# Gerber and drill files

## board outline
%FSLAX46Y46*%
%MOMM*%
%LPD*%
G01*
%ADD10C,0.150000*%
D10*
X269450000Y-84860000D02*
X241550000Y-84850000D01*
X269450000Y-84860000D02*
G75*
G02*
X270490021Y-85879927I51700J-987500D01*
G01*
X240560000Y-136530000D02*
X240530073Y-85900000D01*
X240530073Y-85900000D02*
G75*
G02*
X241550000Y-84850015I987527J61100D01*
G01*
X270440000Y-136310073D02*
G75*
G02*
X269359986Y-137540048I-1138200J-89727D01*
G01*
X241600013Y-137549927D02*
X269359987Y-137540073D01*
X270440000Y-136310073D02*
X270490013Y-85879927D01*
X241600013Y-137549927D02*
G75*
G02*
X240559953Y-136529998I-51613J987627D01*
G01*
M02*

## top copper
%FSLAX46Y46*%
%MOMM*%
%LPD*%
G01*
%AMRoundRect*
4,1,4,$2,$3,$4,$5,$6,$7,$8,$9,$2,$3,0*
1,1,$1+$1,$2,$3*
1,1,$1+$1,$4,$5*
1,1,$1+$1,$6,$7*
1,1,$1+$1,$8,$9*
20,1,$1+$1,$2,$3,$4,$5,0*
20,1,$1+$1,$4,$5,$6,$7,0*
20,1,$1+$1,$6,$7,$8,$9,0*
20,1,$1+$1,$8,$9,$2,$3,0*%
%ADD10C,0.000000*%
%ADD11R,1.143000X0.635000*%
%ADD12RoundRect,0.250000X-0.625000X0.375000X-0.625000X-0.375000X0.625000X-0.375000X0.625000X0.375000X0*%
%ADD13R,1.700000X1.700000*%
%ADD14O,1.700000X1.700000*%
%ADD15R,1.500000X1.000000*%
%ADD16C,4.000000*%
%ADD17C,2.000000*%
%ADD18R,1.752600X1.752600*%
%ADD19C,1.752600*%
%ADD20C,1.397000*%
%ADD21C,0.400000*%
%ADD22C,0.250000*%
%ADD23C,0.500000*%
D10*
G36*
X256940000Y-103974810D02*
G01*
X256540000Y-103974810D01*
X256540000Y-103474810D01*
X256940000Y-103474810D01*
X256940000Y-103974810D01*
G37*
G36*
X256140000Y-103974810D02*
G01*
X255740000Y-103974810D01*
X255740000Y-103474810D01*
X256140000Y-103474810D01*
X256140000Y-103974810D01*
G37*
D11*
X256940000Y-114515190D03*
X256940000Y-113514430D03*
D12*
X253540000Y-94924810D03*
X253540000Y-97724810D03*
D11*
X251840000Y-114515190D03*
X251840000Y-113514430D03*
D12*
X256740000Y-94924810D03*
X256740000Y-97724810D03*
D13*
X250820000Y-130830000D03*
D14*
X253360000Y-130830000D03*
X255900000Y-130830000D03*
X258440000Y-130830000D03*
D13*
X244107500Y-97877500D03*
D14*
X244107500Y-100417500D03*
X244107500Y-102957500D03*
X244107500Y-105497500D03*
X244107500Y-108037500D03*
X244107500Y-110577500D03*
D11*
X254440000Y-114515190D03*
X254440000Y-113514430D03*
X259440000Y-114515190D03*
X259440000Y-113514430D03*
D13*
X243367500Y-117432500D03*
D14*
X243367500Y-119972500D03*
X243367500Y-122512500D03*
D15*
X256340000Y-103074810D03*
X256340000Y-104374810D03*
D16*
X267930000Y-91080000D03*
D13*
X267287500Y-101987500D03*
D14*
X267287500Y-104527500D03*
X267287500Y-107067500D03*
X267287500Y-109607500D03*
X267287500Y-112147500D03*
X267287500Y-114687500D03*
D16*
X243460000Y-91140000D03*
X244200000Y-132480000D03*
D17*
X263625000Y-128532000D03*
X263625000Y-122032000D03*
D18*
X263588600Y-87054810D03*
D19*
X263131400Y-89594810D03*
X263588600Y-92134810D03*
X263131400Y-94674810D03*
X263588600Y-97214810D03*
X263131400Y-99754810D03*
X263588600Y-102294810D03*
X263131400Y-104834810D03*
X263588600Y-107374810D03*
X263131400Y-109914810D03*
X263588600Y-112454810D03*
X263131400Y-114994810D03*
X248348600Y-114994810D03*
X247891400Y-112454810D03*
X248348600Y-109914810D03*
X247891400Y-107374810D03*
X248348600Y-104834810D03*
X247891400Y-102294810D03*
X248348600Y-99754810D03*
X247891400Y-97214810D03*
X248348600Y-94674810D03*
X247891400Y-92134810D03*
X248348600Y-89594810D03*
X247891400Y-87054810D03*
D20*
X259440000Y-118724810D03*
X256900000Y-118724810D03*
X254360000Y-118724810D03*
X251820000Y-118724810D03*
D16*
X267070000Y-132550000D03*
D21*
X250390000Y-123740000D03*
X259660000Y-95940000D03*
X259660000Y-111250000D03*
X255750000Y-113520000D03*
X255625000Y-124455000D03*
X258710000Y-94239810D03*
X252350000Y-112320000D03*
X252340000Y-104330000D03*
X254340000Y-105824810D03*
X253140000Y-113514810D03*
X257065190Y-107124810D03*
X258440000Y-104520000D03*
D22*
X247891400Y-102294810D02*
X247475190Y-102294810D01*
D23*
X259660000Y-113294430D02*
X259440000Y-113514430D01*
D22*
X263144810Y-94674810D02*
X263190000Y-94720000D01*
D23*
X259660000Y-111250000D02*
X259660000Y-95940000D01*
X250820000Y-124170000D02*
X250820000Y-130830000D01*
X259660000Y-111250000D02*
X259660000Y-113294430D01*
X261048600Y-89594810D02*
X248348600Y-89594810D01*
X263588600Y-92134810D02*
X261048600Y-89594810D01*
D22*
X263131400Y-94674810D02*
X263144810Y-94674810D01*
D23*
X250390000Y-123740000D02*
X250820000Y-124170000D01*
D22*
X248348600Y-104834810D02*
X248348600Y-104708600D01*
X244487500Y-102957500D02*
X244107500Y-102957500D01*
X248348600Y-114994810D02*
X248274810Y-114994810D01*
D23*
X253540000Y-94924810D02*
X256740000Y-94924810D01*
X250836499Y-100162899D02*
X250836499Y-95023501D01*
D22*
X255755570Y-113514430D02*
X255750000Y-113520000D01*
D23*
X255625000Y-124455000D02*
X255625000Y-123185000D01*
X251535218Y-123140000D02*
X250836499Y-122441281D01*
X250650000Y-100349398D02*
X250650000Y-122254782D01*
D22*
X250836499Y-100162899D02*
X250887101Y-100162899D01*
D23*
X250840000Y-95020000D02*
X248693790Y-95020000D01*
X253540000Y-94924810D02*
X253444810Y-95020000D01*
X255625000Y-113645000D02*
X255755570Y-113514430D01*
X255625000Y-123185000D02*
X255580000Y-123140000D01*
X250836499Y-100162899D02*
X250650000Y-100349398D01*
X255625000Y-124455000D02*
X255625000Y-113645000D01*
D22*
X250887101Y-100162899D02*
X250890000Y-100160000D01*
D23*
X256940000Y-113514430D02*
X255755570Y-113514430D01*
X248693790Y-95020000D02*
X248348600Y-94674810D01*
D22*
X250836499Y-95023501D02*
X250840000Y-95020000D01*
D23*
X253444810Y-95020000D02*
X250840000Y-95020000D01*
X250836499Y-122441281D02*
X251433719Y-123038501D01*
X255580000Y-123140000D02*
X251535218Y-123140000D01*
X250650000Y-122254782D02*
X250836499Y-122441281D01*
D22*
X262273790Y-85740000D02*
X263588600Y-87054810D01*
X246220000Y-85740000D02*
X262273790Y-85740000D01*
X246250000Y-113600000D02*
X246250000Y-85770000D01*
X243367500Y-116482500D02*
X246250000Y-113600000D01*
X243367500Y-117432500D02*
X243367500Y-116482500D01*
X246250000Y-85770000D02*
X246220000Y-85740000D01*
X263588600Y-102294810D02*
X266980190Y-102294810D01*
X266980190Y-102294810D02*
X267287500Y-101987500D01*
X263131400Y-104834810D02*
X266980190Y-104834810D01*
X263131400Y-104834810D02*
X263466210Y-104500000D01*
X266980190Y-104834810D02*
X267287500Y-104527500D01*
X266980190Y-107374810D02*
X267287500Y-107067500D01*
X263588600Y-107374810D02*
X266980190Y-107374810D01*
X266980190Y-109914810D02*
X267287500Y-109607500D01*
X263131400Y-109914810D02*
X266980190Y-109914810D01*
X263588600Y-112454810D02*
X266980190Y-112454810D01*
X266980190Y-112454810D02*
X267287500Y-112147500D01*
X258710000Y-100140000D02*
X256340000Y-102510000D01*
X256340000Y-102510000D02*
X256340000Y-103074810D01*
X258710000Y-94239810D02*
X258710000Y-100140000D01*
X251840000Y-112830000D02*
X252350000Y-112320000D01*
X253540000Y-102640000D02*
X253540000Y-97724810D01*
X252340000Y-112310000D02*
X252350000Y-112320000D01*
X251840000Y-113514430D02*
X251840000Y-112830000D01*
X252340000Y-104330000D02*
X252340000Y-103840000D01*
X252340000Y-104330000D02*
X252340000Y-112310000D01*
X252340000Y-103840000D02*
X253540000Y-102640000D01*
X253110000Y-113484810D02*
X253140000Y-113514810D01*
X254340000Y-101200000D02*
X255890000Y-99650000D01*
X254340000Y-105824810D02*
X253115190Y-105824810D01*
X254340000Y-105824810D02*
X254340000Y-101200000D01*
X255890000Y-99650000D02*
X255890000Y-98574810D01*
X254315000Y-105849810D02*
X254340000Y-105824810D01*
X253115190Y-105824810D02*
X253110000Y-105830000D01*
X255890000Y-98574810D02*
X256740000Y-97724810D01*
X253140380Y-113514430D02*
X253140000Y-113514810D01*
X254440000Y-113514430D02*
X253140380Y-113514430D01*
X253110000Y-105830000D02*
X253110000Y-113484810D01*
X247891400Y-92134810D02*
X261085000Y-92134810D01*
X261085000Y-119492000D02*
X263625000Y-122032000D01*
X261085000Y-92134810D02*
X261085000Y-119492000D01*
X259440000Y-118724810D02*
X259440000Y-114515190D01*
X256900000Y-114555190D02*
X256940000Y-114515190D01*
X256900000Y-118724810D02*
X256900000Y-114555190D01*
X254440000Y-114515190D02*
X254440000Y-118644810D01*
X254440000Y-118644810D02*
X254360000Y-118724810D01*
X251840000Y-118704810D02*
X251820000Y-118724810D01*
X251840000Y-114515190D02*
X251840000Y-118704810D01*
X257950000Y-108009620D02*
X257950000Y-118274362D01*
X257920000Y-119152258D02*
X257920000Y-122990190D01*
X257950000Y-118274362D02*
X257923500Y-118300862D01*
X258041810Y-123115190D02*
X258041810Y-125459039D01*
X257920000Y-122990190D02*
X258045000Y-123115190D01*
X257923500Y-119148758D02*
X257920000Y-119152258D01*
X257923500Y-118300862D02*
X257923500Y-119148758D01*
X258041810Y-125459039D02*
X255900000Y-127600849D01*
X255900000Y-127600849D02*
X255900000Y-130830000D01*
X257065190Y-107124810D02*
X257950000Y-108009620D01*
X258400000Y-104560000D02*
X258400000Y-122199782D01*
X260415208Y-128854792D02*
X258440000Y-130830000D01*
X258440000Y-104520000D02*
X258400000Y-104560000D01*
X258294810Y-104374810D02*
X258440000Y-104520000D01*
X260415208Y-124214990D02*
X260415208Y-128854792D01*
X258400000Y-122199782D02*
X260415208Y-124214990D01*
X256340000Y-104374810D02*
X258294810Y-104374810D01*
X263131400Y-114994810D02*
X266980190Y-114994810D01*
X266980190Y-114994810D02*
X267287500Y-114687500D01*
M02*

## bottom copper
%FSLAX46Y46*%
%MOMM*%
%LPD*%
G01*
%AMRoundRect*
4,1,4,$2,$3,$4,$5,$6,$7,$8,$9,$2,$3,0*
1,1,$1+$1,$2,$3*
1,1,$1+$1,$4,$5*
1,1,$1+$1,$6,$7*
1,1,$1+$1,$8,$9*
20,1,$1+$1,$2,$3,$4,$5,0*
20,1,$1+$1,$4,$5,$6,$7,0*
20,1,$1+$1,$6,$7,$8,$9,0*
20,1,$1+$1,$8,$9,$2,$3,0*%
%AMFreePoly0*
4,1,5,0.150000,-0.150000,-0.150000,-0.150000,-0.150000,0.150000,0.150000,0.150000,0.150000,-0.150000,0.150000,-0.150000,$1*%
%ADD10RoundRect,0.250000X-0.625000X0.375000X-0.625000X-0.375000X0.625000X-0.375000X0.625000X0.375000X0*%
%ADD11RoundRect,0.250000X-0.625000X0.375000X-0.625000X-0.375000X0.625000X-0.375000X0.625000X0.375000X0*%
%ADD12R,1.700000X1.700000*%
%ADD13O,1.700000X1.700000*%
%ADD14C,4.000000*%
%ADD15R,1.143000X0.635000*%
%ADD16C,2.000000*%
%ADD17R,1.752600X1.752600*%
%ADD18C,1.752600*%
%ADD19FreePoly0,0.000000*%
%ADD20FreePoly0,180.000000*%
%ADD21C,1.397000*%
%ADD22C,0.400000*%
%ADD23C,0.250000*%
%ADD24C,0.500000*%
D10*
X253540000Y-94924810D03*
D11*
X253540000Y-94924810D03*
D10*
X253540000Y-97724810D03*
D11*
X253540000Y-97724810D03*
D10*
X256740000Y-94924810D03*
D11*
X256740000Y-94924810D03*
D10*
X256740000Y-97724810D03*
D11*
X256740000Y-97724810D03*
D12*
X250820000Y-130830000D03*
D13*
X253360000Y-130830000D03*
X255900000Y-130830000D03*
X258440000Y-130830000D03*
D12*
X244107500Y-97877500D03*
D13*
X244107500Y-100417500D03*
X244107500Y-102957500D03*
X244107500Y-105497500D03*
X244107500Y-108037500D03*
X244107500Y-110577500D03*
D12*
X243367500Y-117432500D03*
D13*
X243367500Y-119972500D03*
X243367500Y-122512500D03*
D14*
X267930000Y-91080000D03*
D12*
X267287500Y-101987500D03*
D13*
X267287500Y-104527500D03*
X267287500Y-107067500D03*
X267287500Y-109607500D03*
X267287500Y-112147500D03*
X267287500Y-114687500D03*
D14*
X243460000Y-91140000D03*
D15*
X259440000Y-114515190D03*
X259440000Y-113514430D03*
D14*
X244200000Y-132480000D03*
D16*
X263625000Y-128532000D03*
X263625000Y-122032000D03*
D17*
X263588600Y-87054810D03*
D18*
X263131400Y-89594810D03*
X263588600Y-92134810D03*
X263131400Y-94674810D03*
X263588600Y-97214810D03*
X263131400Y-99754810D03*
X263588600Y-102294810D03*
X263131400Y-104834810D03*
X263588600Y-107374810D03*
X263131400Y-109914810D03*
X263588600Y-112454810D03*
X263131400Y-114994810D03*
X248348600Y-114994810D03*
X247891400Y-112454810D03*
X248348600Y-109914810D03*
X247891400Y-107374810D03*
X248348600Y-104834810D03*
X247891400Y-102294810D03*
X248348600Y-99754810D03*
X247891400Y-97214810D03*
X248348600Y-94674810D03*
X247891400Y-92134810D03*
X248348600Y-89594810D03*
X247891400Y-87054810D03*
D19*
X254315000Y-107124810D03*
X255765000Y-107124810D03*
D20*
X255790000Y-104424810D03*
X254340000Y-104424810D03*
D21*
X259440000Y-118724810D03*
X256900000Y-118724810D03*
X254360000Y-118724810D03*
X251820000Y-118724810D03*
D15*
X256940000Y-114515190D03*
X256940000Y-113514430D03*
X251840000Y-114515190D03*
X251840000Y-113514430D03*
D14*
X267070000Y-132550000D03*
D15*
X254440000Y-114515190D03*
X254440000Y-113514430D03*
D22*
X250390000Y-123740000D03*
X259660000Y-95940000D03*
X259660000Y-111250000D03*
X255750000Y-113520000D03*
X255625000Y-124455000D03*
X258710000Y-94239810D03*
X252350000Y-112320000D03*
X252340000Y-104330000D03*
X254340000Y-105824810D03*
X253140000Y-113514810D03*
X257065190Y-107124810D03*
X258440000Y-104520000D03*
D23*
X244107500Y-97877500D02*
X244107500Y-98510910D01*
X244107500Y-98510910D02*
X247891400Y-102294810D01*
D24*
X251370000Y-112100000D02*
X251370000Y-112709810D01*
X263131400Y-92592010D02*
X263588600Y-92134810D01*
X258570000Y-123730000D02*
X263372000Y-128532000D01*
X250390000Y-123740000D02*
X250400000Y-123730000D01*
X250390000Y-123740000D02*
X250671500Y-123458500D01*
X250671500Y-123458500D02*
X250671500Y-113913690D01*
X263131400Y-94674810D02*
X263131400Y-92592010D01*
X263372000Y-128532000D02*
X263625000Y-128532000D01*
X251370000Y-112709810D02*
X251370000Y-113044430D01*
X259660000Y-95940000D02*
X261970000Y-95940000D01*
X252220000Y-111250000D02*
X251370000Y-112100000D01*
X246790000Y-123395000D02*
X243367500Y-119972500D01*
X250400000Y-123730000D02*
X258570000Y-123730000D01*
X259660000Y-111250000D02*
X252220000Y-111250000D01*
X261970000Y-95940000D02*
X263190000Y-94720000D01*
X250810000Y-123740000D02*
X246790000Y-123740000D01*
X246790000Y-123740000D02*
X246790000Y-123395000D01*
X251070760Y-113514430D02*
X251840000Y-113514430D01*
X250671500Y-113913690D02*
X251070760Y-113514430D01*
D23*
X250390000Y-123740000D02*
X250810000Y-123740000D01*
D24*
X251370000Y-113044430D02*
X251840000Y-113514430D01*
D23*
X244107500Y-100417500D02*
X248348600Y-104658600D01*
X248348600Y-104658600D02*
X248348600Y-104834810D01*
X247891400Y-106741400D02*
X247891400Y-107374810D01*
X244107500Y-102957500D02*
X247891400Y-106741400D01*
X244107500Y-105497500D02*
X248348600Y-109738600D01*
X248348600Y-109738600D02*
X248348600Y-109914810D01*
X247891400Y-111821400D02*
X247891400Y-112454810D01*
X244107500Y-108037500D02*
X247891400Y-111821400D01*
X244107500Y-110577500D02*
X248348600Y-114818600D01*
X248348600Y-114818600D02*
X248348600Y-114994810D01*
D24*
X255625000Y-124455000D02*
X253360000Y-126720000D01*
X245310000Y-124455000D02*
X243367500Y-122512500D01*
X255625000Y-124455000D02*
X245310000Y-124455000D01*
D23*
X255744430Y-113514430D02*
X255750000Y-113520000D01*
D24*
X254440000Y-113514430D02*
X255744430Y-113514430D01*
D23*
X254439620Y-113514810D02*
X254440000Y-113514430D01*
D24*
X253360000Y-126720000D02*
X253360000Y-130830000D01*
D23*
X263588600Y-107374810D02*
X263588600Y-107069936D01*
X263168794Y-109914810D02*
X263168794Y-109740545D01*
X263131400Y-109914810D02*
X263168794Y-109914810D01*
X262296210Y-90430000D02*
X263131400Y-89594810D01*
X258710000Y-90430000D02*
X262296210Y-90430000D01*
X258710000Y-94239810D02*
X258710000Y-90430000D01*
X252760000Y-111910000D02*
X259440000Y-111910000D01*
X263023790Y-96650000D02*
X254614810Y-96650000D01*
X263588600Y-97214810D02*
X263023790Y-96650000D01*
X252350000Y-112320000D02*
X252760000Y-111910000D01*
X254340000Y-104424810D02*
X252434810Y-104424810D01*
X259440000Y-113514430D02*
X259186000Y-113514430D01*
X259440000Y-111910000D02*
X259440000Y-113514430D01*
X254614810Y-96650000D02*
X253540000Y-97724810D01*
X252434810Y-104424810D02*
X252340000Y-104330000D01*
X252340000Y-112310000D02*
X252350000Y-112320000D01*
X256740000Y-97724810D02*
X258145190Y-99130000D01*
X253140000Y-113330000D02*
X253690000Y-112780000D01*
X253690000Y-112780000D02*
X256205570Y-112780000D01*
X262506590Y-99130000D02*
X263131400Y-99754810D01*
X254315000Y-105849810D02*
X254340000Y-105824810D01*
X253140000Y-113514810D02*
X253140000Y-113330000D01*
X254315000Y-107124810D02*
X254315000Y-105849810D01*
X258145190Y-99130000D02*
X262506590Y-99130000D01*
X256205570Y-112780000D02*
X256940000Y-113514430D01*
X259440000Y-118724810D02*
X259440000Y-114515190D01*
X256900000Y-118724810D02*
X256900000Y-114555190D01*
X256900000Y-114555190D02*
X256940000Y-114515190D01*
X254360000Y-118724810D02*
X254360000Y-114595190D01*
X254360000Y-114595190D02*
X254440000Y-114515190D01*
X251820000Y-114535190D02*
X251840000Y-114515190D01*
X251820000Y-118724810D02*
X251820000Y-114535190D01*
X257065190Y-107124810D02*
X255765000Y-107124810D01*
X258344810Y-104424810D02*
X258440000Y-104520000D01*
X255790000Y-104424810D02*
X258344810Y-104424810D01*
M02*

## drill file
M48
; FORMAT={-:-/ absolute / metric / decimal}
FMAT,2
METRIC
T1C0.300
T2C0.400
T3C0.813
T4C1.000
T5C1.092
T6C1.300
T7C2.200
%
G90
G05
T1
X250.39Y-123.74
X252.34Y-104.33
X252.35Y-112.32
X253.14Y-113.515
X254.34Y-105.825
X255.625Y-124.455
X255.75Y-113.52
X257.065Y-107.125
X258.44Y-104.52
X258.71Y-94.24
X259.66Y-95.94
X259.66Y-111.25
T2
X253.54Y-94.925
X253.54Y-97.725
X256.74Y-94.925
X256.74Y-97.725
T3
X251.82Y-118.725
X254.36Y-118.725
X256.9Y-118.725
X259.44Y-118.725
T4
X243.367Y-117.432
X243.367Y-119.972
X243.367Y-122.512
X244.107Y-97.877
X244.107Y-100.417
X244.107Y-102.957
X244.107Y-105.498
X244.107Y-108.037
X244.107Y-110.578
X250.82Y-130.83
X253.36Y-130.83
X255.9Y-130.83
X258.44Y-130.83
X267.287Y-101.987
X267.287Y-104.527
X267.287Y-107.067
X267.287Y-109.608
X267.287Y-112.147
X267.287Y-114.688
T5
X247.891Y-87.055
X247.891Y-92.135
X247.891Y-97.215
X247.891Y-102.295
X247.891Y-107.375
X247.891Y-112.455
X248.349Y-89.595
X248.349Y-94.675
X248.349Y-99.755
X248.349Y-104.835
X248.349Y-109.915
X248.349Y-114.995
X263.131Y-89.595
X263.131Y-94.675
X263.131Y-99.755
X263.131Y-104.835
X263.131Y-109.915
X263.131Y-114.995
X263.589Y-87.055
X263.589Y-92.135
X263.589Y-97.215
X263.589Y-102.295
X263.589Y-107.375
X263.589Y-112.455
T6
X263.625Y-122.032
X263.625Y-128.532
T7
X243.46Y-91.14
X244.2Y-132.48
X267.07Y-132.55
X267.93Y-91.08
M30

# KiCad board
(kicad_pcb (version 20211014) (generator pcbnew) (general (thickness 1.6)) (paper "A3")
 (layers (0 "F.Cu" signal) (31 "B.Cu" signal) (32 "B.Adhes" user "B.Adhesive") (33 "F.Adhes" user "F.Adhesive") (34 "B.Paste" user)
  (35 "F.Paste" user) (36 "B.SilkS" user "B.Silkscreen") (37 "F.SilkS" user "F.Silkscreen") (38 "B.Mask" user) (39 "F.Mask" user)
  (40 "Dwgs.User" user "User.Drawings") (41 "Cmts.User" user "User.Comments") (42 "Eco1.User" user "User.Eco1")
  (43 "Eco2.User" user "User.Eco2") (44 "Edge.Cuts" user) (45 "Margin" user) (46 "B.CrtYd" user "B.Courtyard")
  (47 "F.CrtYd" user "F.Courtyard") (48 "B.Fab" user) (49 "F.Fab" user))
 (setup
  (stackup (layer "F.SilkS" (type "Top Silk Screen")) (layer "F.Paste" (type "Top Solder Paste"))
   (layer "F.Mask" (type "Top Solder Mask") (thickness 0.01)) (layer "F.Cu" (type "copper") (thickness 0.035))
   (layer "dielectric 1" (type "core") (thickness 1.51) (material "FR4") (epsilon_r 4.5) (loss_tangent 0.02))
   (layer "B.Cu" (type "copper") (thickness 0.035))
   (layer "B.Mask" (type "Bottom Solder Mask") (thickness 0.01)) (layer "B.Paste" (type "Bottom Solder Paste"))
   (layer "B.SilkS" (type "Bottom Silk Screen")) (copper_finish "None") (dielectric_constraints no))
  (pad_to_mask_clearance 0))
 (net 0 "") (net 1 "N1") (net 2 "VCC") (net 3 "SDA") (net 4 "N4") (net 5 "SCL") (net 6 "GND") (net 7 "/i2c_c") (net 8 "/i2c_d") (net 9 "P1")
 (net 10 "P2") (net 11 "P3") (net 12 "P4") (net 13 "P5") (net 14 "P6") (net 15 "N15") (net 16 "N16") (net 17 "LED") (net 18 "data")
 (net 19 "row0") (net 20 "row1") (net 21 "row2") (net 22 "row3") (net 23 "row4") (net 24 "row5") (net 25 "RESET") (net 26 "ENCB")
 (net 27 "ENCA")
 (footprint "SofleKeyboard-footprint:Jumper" (layer "F.Cu") (at 256.94 114.01481 90)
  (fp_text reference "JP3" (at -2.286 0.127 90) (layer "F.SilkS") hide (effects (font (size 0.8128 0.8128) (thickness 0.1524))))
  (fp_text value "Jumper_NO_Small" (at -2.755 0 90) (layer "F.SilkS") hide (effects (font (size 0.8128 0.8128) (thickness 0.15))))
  (pad "1" smd rect locked (at -0.50038 0 90) (size 0.635 1.143) (layers "F.Cu" "F.Paste" "F.Mask") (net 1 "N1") (clearance 0.1905))
  (pad "2" smd rect locked (at 0.50038 0 90) (size 0.635 1.143) (layers "F.Cu" "F.Paste" "F.Mask") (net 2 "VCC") (clearance 0.1905)))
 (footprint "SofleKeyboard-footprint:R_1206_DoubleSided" (layer "F.Cu") (at 253.54 96.32481 -90)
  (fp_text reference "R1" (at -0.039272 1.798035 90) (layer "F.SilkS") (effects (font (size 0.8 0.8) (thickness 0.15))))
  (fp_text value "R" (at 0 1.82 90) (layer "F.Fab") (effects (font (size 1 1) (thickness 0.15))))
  (pad "1" thru_hole roundrect locked (at -1.4 0 270) (size 1.25 1.75) (drill 0.4) (layers F&B.Cu *.Mask) (roundrect_rratio 0.2)
   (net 2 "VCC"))
  (pad "1" smd roundrect locked (at -1.4 0 270) (size 1.25 1.75) (layers "B.Cu" "B.Paste" "B.Mask") (roundrect_rratio 0.2) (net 2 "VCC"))
  (pad "2" thru_hole roundrect locked (at 1.4 0 270) (size 1.25 1.75) (drill 0.4) (layers *.Cu *.Mask) (roundrect_rratio 0.2) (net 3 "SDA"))
  (pad "2" smd roundrect locked (at 1.4 0 270) (size 1.25 1.75) (layers "B.Cu" "B.Paste" "B.Mask") (roundrect_rratio 0.2) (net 3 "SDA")))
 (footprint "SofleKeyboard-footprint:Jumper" (layer "F.Cu") (at 251.84 114.01481 90)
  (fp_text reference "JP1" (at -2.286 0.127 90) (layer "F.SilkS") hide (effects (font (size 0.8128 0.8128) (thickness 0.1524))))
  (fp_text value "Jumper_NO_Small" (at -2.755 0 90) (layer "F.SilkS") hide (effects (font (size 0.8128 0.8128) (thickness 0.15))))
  (pad "1" smd rect locked (at -0.50038 0 90) (size 0.635 1.143) (layers "F.Cu" "F.Paste" "F.Mask") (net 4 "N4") (clearance 0.1905))
  (pad "2" smd rect locked (at 0.50038 0 90) (size 0.635 1.143) (layers "F.Cu" "F.Paste" "F.Mask") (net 3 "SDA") (clearance 0.1905)))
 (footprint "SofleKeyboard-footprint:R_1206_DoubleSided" (layer "F.Cu") (at 256.74 96.32481 -90)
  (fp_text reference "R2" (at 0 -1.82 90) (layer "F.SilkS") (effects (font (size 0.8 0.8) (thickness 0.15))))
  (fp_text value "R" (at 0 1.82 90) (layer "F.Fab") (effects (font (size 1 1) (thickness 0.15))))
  (pad "1" thru_hole roundrect locked (at -1.4 0 270) (size 1.25 1.75) (drill 0.4) (layers F&B.Cu *.Mask) (roundrect_rratio 0.2)
   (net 2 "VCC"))
  (pad "1" smd roundrect locked (at -1.4 0 270) (size 1.25 1.75) (layers "B.Cu" "B.Paste" "B.Mask") (roundrect_rratio 0.2) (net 2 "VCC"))
  (pad "2" thru_hole roundrect locked (at 1.4 0 270) (size 1.25 1.75) (drill 0.4) (layers *.Cu *.Mask) (roundrect_rratio 0.2) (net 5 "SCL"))
  (pad "2" smd roundrect locked (at 1.4 0 270) (size 1.25 1.75) (layers "B.Cu" "B.Paste" "B.Mask") (roundrect_rratio 0.2) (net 5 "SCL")))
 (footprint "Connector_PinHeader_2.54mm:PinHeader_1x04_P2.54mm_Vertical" (layer "F.Cu") (at 250.82 130.83 90)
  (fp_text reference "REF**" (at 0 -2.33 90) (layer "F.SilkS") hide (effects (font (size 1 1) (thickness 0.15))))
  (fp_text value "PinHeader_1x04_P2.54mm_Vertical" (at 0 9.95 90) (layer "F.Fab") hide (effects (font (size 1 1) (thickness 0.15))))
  (pad "1" thru_hole rect (at 0 0 90) (size 1.7 1.7) (drill 1) (layers F&B.Cu *.Mask) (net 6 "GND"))
  (pad "2" thru_hole oval (at 0 2.54 90) (size 1.7 1.7) (drill 1) (layers F&B.Cu *.Mask) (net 2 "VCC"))
  (pad "3" thru_hole oval (at 0 5.08 90) (size 1.7 1.7) (drill 1) (layers F&B.Cu *.Mask) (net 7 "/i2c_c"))
  (pad "4" thru_hole oval (at 0 7.62 90) (size 1.7 1.7) (drill 1) (layers F&B.Cu *.Mask) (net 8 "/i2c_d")))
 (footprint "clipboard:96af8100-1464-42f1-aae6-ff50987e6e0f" (layer "F.Cu") (at 245.9075 112.3775)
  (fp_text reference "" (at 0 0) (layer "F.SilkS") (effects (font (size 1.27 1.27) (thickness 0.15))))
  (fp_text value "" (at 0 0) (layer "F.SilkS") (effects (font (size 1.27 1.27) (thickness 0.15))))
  (pad "1" thru_hole rect (at -1.8 -14.5) (size 1.7 1.7) (drill 1) (layers F&B.Cu *.Mask) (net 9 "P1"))
  (pad "2" thru_hole oval (at -1.8 -11.96) (size 1.7 1.7) (drill 1) (layers F&B.Cu *.Mask) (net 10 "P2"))
  (pad "3" thru_hole oval (at -1.8 -9.42) (size 1.7 1.7) (drill 1) (layers F&B.Cu *.Mask) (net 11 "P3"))
  (pad "4" thru_hole oval (at -1.8 -6.88) (size 1.7 1.7) (drill 1) (layers F&B.Cu *.Mask) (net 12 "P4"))
  (pad "5" thru_hole oval (at -1.8 -4.34) (size 1.7 1.7) (drill 1) (layers F&B.Cu *.Mask) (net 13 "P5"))
  (pad "6" thru_hole oval (at -1.8 -1.8) (size 1.7 1.7) (drill 1) (layers F&B.Cu *.Mask) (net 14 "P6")))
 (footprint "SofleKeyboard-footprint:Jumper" (layer "F.Cu") (at 254.44 114.01481 90)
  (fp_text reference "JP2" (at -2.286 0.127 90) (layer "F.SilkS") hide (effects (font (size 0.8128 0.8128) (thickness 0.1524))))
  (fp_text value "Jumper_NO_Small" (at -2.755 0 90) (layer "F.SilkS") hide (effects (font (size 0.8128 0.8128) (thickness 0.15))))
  (pad "1" smd rect locked (at -0.50038 0 90) (size 0.635 1.143) (layers "F.Cu" "F.Paste" "F.Mask") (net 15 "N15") (clearance 0.1905))
  (pad "2" smd rect locked (at 0.50038 0 90) (size 0.635 1.143) (layers "F.Cu" "F.Paste" "F.Mask") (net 5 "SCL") (clearance 0.1905)))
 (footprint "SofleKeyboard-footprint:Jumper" (layer "F.Cu") (at 259.44 114.01481 90)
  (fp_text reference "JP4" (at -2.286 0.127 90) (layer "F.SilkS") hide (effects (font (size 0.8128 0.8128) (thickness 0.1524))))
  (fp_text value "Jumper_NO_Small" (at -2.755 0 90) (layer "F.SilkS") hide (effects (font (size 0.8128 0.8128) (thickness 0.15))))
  (pad "1" smd rect locked (at -0.50038 0 90) (size 0.635 1.143) (layers "F.Cu" "F.Paste" "F.Mask") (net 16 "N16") (clearance 0.1905))
  (pad "2" smd rect locked (at 0.50038 0 90) (size 0.635 1.143) (layers "F.Cu" "F.Paste" "F.Mask") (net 6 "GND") (clearance 0.1905)))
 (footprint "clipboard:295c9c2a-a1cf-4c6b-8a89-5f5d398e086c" (layer "F.Cu") (at 245.1675 124.2825)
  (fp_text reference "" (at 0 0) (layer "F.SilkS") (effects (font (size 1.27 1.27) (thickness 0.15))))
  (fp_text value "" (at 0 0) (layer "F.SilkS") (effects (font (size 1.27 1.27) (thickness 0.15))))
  (pad "1" thru_hole rect (at -1.8 -6.85) (size 1.7 1.7) (drill 1) (layers F&B.Cu *.Mask) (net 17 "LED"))
  (pad "2" thru_hole oval (at -1.8 -4.31) (size 1.7 1.7) (drill 1) (layers F&B.Cu *.Mask) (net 6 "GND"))
  (pad "3" thru_hole oval (at -1.8 -1.77) (size 1.7 1.7) (drill 1) (layers F&B.Cu *.Mask) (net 2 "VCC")))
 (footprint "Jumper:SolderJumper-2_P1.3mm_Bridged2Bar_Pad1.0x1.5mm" (layer "F.Cu") (at 256.34 103.72481 -90)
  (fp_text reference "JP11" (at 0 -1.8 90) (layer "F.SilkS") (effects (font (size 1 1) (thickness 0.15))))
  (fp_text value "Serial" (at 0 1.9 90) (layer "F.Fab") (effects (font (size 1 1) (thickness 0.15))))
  (fp_poly (pts (xy -0.25 -0.6) (xy 0.25 -0.6) (xy 0.25 -0.2) (xy -0.25 -0.2)) (layer "F.Cu") (width 0) (fill solid))
  (fp_poly (pts (xy -0.25 0.2) (xy 0.25 0.2) (xy 0.25 0.6) (xy -0.25 0.6)) (layer "F.Cu") (width 0) (fill solid))
  (pad "1" smd rect locked (at -0.65 0 270) (size 1 1.5) (layers "F.Cu" "F.Mask") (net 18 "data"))
  (pad "2" smd rect locked (at 0.65 0 270) (size 1 1.5) (layers "F.Cu" "F.Mask") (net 8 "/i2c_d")))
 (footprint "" (layer "F.Cu") (at 267.93 91.08)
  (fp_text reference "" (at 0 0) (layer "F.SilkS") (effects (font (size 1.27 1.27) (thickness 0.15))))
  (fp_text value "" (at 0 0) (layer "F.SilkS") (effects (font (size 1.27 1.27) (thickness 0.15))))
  (pad "" thru_hole circle locked (at 0 0 180) (size 4 4) (drill 2.2) (layers F&B.Cu *.Mask "Dwgs.User")))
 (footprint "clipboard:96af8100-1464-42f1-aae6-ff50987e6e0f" (layer "F.Cu") (at 269.0875 116.4875)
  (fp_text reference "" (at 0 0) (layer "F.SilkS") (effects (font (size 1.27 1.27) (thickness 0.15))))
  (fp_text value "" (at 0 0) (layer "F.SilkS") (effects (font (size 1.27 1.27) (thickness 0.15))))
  (pad "1" thru_hole rect (at -1.8 -14.5) (size 1.7 1.7) (drill 1) (layers F&B.Cu *.Mask) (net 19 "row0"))
  (pad "2" thru_hole oval (at -1.8 -11.96) (size 1.7 1.7) (drill 1) (layers F&B.Cu *.Mask) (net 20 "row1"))
  (pad "3" thru_hole oval (at -1.8 -9.42) (size 1.7 1.7) (drill 1) (layers F&B.Cu *.Mask) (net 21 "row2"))
  (pad "4" thru_hole oval (at -1.8 -6.88) (size 1.7 1.7) (drill 1) (layers F&B.Cu *.Mask) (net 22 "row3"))
  (pad "5" thru_hole oval (at -1.8 -4.34) (size 1.7 1.7) (drill 1) (layers F&B.Cu *.Mask) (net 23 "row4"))
  (pad "6" thru_hole oval (at -1.8 -1.8) (size 1.7 1.7) (drill 1) (layers F&B.Cu *.Mask) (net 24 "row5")))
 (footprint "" (layer "F.Cu") (at 243.46 91.14)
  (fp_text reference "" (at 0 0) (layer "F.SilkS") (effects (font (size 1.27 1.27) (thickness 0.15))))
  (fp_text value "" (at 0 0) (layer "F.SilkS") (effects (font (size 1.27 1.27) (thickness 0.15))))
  (pad "" thru_hole circle locked (at 0 0 180) (size 4 4) (drill 2.2) (layers F&B.Cu *.Mask "Dwgs.User")))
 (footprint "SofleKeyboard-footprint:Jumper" (layer "B.Cu") (at 259.44 114.01481 90)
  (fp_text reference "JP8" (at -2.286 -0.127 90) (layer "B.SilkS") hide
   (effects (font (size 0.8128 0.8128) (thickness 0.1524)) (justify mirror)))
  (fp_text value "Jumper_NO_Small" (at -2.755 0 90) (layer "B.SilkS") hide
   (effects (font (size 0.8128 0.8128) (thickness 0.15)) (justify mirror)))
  (pad "1" smd rect locked (at -0.50038 0 90) (size 0.635 1.143) (layers "B.Cu" "B.Paste" "B.Mask") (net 16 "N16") (clearance 0.1905))
  (pad "2" smd rect locked (at 0.50038 0 90) (size 0.635 1.143) (layers "B.Cu" "B.Paste" "B.Mask") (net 3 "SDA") (clearance 0.1905)))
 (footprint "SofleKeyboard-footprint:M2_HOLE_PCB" (layer "B.Cu") (at 244.2 132.48 180)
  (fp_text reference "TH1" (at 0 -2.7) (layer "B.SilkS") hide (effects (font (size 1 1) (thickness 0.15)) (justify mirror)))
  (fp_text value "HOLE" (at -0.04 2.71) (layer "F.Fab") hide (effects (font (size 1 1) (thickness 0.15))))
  (pad "" thru_hole circle locked (at 0 0 180) (size 4 4) (drill 2.2) (layers F&B.Cu *.Mask "Dwgs.User")))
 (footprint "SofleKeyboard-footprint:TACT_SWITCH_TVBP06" (layer "B.Cu") (at 263.625 125.282 90)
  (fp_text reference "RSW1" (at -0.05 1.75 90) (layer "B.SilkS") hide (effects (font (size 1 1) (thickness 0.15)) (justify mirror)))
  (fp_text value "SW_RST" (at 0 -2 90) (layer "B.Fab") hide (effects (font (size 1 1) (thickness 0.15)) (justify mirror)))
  (pad "1" thru_hole circle locked (at -3.25 0 90) (size 2 2) (drill 1.3) (layers F&B.Cu *.Mask) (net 6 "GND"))
  (pad "2" thru_hole circle locked (at 3.25 0 90) (size 2 2) (drill 1.3) (layers *.Cu *.Mask) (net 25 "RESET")))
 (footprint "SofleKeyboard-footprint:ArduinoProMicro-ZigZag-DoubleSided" (layer "B.Cu") (at 255.74 101.02481 -90)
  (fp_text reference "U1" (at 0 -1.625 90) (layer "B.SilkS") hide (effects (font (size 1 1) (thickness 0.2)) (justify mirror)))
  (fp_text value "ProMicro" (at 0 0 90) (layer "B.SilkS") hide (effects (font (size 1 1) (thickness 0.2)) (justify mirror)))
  (pad "1" thru_hole rect locked (at -13.97 -7.8486 270) (size 1.7526 1.7526) (drill 1.0922) (layers *.Cu *.SilkS *.Mask) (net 17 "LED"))
  (pad "2" thru_hole circle locked (at -11.43 -7.3914 270) (size 1.7526 1.7526) (drill 1.0922) (layers *.Cu *.SilkS *.Mask) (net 18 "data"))
  (pad "3" thru_hole circle locked (at -8.89 -7.8486 270) (size 1.7526 1.7526) (drill 1.0922) (layers F&B.Cu *.SilkS *.Mask) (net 6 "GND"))
  (pad "4" thru_hole circle locked (at -6.35 -7.3914 270) (size 1.7526 1.7526) (drill 1.0922) (layers F&B.Cu *.SilkS *.Mask) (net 6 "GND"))
  (pad "5" thru_hole circle locked (at -3.81 -7.8486 270) (size 1.7526 1.7526) (drill 1.0922) (layers *.Cu *.SilkS *.Mask) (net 3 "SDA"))
  (pad "6" thru_hole circle locked (at -1.27 -7.3914 270) (size 1.7526 1.7526) (drill 1.0922) (layers *.Cu *.SilkS *.Mask) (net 5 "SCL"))
  (pad "7" thru_hole circle locked (at 1.27 -7.8486 270) (size 1.7526 1.7526) (drill 1.0922) (layers *.Cu *.SilkS *.Mask) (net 19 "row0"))
  (pad "8" thru_hole circle locked (at 3.81 -7.3914 270) (size 1.7526 1.7526) (drill 1.0922) (layers *.Cu *.SilkS *.Mask) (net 20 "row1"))
  (pad "9" thru_hole circle locked (at 6.35 -7.8486 270) (size 1.7526 1.7526) (drill 1.0922) (layers *.Cu *.SilkS *.Mask) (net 21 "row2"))
  (pad "10" thru_hole circle locked (at 8.89 -7.3914 270) (size 1.7526 1.7526) (drill 1.0922) (layers *.Cu *.SilkS *.Mask) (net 22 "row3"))
  (pad "11" thru_hole circle locked (at 11.43 -7.8486 270) (size 1.7526 1.7526) (drill 1.0922) (layers *.Cu *.SilkS *.Mask) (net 23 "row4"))
  (pad "12" thru_hole circle locked (at 13.97 -7.3914 270) (size 1.7526 1.7526) (drill 1.0922) (layers *.Cu *.SilkS *.Mask) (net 24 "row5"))
  (pad "13" thru_hole circle locked (at 13.97 7.3914 270) (size 1.7526 1.7526) (drill 1.0922) (layers *.Cu *.SilkS *.Mask) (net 14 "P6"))
  (pad "14" thru_hole circle locked (at 11.43 7.8486 270) (size 1.7526 1.7526) (drill 1.0922) (layers *.Cu *.SilkS *.Mask) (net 13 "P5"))
  (pad "15" thru_hole circle locked (at 8.89 7.3914 270) (size 1.7526 1.7526) (drill 1.0922) (layers *.Cu *.SilkS *.Mask) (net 12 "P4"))
  (pad "16" thru_hole circle locked (at 6.35 7.8486 270) (size 1.7526 1.7526) (drill 1.0922) (layers *.Cu *.SilkS *.Mask) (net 11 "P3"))
  (pad "17" thru_hole circle locked (at 3.81 7.3914 270) (size 1.7526 1.7526) (drill 1.0922) (layers *.Cu *.SilkS *.Mask) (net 10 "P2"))
  (pad "18" thru_hole circle locked (at 1.27 7.8486 270) (size 1.7526 1.7526) (drill 1.0922) (layers *.Cu *.SilkS *.Mask) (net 9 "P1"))
  (pad "19" thru_hole circle locked (at -1.27 7.3914 270) (size 1.7526 1.7526) (drill 1.0922) (layers *.Cu *.SilkS *.Mask) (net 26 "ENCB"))
  (pad "20" thru_hole circle locked (at -3.81 7.8486 270) (size 1.7526 1.7526) (drill 1.0922) (layers *.Cu *.SilkS *.Mask) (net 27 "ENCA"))
  (pad "21" thru_hole circle locked (at -6.35 7.3914 270) (size 1.7526 1.7526) (drill 1.0922) (layers F&B.Cu *.SilkS *.Mask) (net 2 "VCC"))
  (pad "22" thru_hole circle locked (at -8.89 7.8486 270) (size 1.7526 1.7526) (drill 1.0922) (layers *.Cu *.SilkS *.Mask) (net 25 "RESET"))
  (pad "23" thru_hole circle locked (at -11.43 7.3914 270) (size 1.7526 1.7526) (drill 1.0922) (layers F&B.Cu *.SilkS *.Mask) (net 6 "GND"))
  (pad "24" thru_hole circle locked (at -13.97 7.8486 270) (size 1.7526 1.7526) (drill 1.0922) (layers F&B.Cu *.SilkS *.Mask)))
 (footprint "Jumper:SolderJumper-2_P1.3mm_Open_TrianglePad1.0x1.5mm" (layer "B.Cu") (at 255.04 107.12481)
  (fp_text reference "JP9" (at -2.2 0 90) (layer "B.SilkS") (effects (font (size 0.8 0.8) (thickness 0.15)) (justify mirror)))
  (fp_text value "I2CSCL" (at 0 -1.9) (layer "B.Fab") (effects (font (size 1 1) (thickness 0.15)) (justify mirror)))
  (pad "1" smd custom locked (at -0.725 0) (size 0.3 0.3) (layers "B.Cu" "B.Mask") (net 5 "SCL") (zone_connect 2)
   (options (clearance outline) (anchor rect)) (primitives))
  (pad "2" smd custom locked (at 0.725 0) (size 0.3 0.3) (layers "B.Cu" "B.Mask") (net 7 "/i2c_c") (zone_connect 2)
   (options (clearance outline) (anchor rect)) (primitives)))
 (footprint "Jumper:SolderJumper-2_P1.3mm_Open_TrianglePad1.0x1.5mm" (layer "B.Cu") (at 255.065 104.42481 180)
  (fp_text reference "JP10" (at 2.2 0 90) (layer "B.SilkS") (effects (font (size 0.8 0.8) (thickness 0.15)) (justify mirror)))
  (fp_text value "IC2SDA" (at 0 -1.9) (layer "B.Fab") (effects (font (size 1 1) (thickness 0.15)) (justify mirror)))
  (pad "1" smd custom locked (at -0.725 0 180) (size 0.3 0.3) (layers "B.Cu" "B.Mask") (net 8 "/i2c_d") (zone_connect 2)
   (options (clearance outline) (anchor rect)) (primitives))
  (pad "2" smd custom locked (at 0.725 0 180) (size 0.3 0.3) (layers "B.Cu" "B.Mask") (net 3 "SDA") (zone_connect 2)
   (options (clearance outline) (anchor rect)) (primitives)))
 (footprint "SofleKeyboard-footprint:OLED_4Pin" (layer "B.Cu") (at 259.44 118.72481 180)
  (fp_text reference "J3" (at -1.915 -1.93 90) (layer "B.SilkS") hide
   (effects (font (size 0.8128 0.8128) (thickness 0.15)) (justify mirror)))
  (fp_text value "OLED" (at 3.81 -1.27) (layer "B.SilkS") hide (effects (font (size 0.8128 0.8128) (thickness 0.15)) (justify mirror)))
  (pad "1" thru_hole circle locked (at 0 0 180) (size 1.397 1.397) (drill 0.8128) (layers *.Cu *.Mask "B.SilkS") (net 16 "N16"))
  (pad "2" thru_hole circle locked (at 2.54 0 180) (size 1.397 1.397) (drill 0.8128) (layers *.Cu *.Mask "B.SilkS") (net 1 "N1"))
  (pad "3" thru_hole circle locked (at 5.08 0 180) (size 1.397 1.397) (drill 0.8128) (layers *.Cu *.Mask "B.SilkS") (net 15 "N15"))
  (pad "4" thru_hole circle locked (at 7.62 0 180) (size 1.397 1.397) (drill 0.8128) (layers *.Cu *.Mask "B.SilkS") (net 4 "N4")))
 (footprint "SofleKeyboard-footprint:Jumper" (layer "B.Cu") (at 256.94 114.01481 90)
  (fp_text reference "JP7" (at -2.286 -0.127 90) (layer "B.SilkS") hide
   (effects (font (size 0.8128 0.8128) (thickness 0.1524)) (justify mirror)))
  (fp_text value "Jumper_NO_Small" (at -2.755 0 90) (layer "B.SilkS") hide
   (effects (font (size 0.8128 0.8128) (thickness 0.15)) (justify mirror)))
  (pad "1" smd rect locked (at -0.50038 0 90) (size 0.635 1.143) (layers "B.Cu" "B.Paste" "B.Mask") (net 1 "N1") (clearance 0.1905))
  (pad "2" smd rect locked (at 0.50038 0 90) (size 0.635 1.143) (layers "B.Cu" "B.Paste" "B.Mask") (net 5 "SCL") (clearance 0.1905)))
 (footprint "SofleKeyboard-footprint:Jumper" (layer "B.Cu") (at 251.84 114.01481 90)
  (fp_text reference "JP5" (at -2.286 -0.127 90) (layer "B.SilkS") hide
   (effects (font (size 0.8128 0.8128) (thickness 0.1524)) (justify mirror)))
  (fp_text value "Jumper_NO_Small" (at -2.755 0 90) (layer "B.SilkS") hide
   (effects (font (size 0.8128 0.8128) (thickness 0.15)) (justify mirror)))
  (pad "1" smd rect locked (at -0.50038 0 90) (size 0.635 1.143) (layers "B.Cu" "B.Paste" "B.Mask") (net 4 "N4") (clearance 0.1905))
  (pad "2" smd rect locked (at 0.50038 0 90) (size 0.635 1.143) (layers "B.Cu" "B.Paste" "B.Mask") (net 6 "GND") (clearance 0.1905)))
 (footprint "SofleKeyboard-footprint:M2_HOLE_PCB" (layer "B.Cu") (at 267.07 132.55 180)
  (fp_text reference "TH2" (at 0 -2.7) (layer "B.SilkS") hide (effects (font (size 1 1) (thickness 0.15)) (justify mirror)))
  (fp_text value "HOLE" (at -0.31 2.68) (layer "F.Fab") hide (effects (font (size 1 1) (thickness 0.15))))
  (pad "" thru_hole circle locked (at 0 0 180) (size 4 4) (drill 2.2) (layers F&B.Cu *.Mask "Dwgs.User")))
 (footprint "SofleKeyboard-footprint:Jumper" (layer "B.Cu") (at 254.44 114.01481 90)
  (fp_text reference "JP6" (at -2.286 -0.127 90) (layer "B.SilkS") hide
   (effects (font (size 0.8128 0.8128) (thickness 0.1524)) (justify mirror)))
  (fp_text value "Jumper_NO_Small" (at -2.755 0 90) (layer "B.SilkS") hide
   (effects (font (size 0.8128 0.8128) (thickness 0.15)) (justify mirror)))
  (pad "1" smd rect locked (at -0.50038 0 90) (size 0.635 1.143) (layers "B.Cu" "B.Paste" "B.Mask") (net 15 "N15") (clearance 0.1905))
  (pad "2" smd rect locked (at 0.50038 0 90) (size 0.635 1.143) (layers "B.Cu" "B.Paste" "B.Mask") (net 2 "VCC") (clearance 0.1905)))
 (gr_line (start 269.45 84.86) (end 241.55 84.85) (layer "Edge.Cuts") (width 0.15))
 (gr_arc (start 269.45 84.86) (mid 270.194055 85.141502) (end 270.490013 85.879927) (layer "Edge.Cuts") (width 0.15))
 (gr_line (start 240.56 136.53) (end 240.530073 85.9) (layer "Edge.Cuts") (width 0.15))
 (gr_arc (start 240.530073 85.9) (mid 240.80788 85.149493) (end 241.55 84.85) (layer "Edge.Cuts") (width 0.15))
 (gr_arc (start 270.44 136.310073) (mid 270.15974 137.153146) (end 269.359987 137.540073) (layer "Edge.Cuts") (width 0.15))
 (gr_line (start 241.600013 137.549927) (end 269.359987 137.540073) (layer "Edge.Cuts") (width 0.15))
 (gr_line (start 270.44 136.310073) (end 270.490013 85.879927) (layer "Edge.Cuts") (width 0.15))
 (gr_arc (start 241.600013 137.549927) (mid 240.855993 137.268407) (end 240.56 136.53) (layer "Edge.Cuts") (width 0.15))
 (segment (start 247.8914 102.29481) (end 247.47519 102.29481) (width 0.25) (layer "F.Cu") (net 9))
 (segment (start 244.1075 97.8775) (end 244.1075 98.51091) (width 0.25) (layer "B.Cu") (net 9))
 (segment (start 244.1075 98.51091) (end 247.8914 102.29481) (width 0.25) (layer "B.Cu") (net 9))
 (segment (start 259.66 113.29443) (end 259.44 113.51443) (width 0.5) (layer "F.Cu") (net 6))
 (segment (start 263.14481 94.67481) (end 263.19 94.72) (width 0.25) (layer "F.Cu") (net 6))
 (segment (start 259.66 111.25) (end 259.66 95.94) (width 0.5) (layer "F.Cu") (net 6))
 (segment (start 250.82 124.17) (end 250.82 130.83) (width 0.5) (layer "F.Cu") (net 6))
 (segment (start 259.66 111.25) (end 259.66 113.29443) (width 0.5) (layer "F.Cu") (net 6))
 (segment (start 261.0486 89.59481) (end 248.3486 89.59481) (width 0.5) (layer "F.Cu") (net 6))
 (segment (start 263.5886 92.13481) (end 261.0486 89.59481) (width 0.5) (layer "F.Cu") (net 6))
 (segment (start 263.1314 94.67481) (end 263.14481 94.67481) (width 0.25) (layer "F.Cu") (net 6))
 (segment (start 250.39 123.74) (end 250.82 124.17) (width 0.5) (layer "F.Cu") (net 6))
 (via (at 250.39 123.74) (size 0.4) (drill 0.3) (layers "F.Cu" "B.Cu") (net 6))
 (via (at 259.66 95.94) (size 0.4) (drill 0.3) (layers "F.Cu" "B.Cu") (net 6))
 (via (at 259.66 111.25) (size 0.4) (drill 0.3) (layers "F.Cu" "B.Cu") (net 6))
 (segment (start 251.37 112.1) (end 251.37 112.70981) (width 0.5) (layer "B.Cu") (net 6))
 (segment (start 263.1314 92.59201) (end 263.5886 92.13481) (width 0.5) (layer "B.Cu") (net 6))
 (segment (start 258.57 123.73) (end 263.372 128.532) (width 0.5) (layer "B.Cu") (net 6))
 (segment (start 250.39 123.74) (end 250.4 123.73) (width 0.5) (layer "B.Cu") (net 6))
 (segment (start 250.39 123.74) (end 250.6715 123.4585) (width 0.5) (layer "B.Cu") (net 6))
 (segment (start 250.6715 123.4585) (end 250.6715 113.91369) (width 0.5) (layer "B.Cu") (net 6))
 (segment (start 263.1314 94.67481) (end 263.1314 92.59201) (width 0.5) (layer "B.Cu") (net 6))
 (segment (start 263.372 128.532) (end 263.625 128.532) (width 0.5) (layer "B.Cu") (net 6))
 (segment (start 251.37 112.70981) (end 251.37 113.04443) (width 0.5) (layer "B.Cu") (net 6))
 (segment (start 259.66 95.94) (end 261.97 95.94) (width 0.5) (layer "B.Cu") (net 6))
 (segment (start 252.22 111.25) (end 251.37 112.1) (width 0.5) (layer "B.Cu") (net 6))
 (segment (start 246.79 123.395) (end 243.3675 119.9725) (width 0.5) (layer "B.Cu") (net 6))
 (segment (start 250.4 123.73) (end 258.57 123.73) (width 0.5) (layer "B.Cu") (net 6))
 (segment (start 259.66 111.25) (end 252.22 111.25) (width 0.5) (layer "B.Cu") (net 6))
 (segment (start 261.97 95.94) (end 263.19 94.72) (width 0.5) (layer "B.Cu") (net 6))
 (segment (start 250.81 123.74) (end 246.79 123.74) (width 0.5) (layer "B.Cu") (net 6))
 (segment (start 246.79 123.74) (end 246.79 123.395) (width 0.5) (layer "B.Cu") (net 6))
 (segment (start 251.07076 113.51443) (end 251.84 113.51443) (width 0.5) (layer "B.Cu") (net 6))
 (segment (start 250.6715 113.91369) (end 251.07076 113.51443) (width 0.5) (layer "B.Cu") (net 6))
 (segment (start 250.39 123.74) (end 250.81 123.74) (width 0.25) (layer "B.Cu") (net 6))
 (segment (start 251.37 113.04443) (end 251.84 113.51443) (width 0.5) (layer "B.Cu") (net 6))
 (segment (start 248.3486 104.83481) (end 248.3486 104.7086) (width 0.25) (layer "F.Cu") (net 10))
 (segment (start 244.1075 100.4175) (end 248.3486 104.6586) (width 0.25) (layer "B.Cu") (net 10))
 (segment (start 248.3486 104.6586) (end 248.3486 104.83481) (width 0.25) (layer "B.Cu") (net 10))
 (segment (start 244.4875 102.9575) (end 244.1075 102.9575) (width 0.25) (layer "F.Cu") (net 11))
 (segment (start 247.8914 106.7414) (end 247.8914 107.37481) (width 0.25) (layer "B.Cu") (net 11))
 (segment (start 244.1075 102.9575) (end 247.8914 106.7414) (width 0.25) (layer "B.Cu") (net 11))
 (segment (start 244.1075 105.4975) (end 248.3486 109.7386) (width 0.25) (layer "B.Cu") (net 12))
 (segment (start 248.3486 109.7386) (end 248.3486 109.91481) (width 0.25) (layer "B.Cu") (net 12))
 (segment (start 247.8914 111.8214) (end 247.8914 112.45481) (width 0.25) (layer "B.Cu") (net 13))
 (segment (start 244.1075 108.0375) (end 247.8914 111.8214) (width 0.25) (layer "B.Cu") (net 13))
 (segment (start 248.3486 114.99481) (end 248.27481 114.99481) (width 0.25) (layer "F.Cu") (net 14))
 (segment (start 244.1075 110.5775) (end 248.3486 114.8186) (width 0.25) (layer "B.Cu") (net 14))
 (segment (start 248.3486 114.8186) (end 248.3486 114.99481) (width 0.25) (layer "B.Cu") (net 14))
 (segment (start 253.54 94.92481) (end 256.74 94.92481) (width 0.5) (layer "F.Cu") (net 2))
 (segment (start 250.836499 100.162899) (end 250.836499 95.023501) (width 0.5) (layer "F.Cu") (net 2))
 (segment (start 255.75557 113.51443) (end 255.75 113.52) (width 0.25) (layer "F.Cu") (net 2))
 (segment (start 255.625 124.455) (end 255.625 123.185) (width 0.5) (layer "F.Cu") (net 2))
 (segment (start 251.535218 123.14) (end 250.836499 122.441281) (width 0.5) (layer "F.Cu") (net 2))
 (segment (start 250.65 100.349398) (end 250.65 122.254782) (width 0.5) (layer "F.Cu") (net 2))
 (segment (start 250.836499 100.162899) (end 250.887101 100.162899) (width 0.25) (layer "F.Cu") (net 2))
 (segment (start 250.84 95.02) (end 248.69379 95.02) (width 0.5) (layer "F.Cu") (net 2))
 (segment (start 253.54 94.92481) (end 253.44481 95.02) (width 0.5) (layer "F.Cu") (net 2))
 (segment (start 255.625 113.645) (end 255.75557 113.51443) (width 0.5) (layer "F.Cu") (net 2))
 (segment (start 255.625 123.185) (end 255.58 123.14) (width 0.5) (layer "F.Cu") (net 2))
 (segment (start 250.836499 100.162899) (end 250.65 100.349398) (width 0.5) (layer "F.Cu") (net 2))
 (segment (start 255.625 124.455) (end 255.625 113.645) (width 0.5) (layer "F.Cu") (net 2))
 (segment (start 250.887101 100.162899) (end 250.89 100.16) (width 0.25) (layer "F.Cu") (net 2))
 (segment (start 256.94 113.51443) (end 255.75557 113.51443) (width 0.5) (layer "F.Cu") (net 2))
 (segment (start 248.69379 95.02) (end 248.3486 94.67481) (width 0.5) (layer "F.Cu") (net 2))
 (segment (start 250.836499 95.023501) (end 250.84 95.02) (width 0.25) (layer "F.Cu") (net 2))
 (segment (start 253.44481 95.02) (end 250.84 95.02) (width 0.5) (layer "F.Cu") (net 2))
 (segment (start 250.836499 122.441281) (end 251.433719 123.038501) (width 0.5) (layer "F.Cu") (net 2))
 (segment (start 255.58 123.14) (end 251.535218 123.14) (width 0.5) (layer "F.Cu") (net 2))
 (segment (start 250.65 122.254782) (end 250.836499 122.441281) (width 0.5) (layer "F.Cu") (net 2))
 (via (at 255.75 113.52) (size 0.4) (drill 0.3) (layers "F.Cu" "B.Cu") (free) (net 2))
 (via (at 255.625 124.455) (size 0.4) (drill 0.3) (layers "F.Cu" "B.Cu") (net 2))
 (segment (start 255.625 124.455) (end 253.36 126.72) (width 0.5) (layer "B.Cu") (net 2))
 (segment (start 245.31 124.455) (end 243.3675 122.5125) (width 0.5) (layer "B.Cu") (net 2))
 (segment (start 255.625 124.455) (end 245.31 124.455) (width 0.5) (layer "B.Cu") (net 2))
 (segment (start 255.74443 113.51443) (end 255.75 113.52) (width 0.25) (layer "B.Cu") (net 2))
 (segment (start 254.44 113.51443) (end 255.74443 113.51443) (width 0.5) (layer "B.Cu") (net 2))
 (segment (start 254.43962 113.51481) (end 254.44 113.51443) (width 0.25) (layer "B.Cu") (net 2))
 (segment (start 253.36 126.72) (end 253.36 130.83) (width 0.5) (layer "B.Cu") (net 2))
 (segment (start 262.27379 85.74) (end 263.5886 87.05481) (width 0.25) (layer "F.Cu") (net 17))
 (segment (start 246.22 85.74) (end 262.27379 85.74) (width 0.25) (layer "F.Cu") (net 17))
 (segment (start 246.25 113.6) (end 246.25 85.77) (width 0.25) (layer "F.Cu") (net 17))
 (segment (start 243.3675 116.4825) (end 246.25 113.6) (width 0.25) (layer "F.Cu") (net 17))
 (segment (start 243.3675 117.4325) (end 243.3675 116.4825) (width 0.25) (layer "F.Cu") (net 17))
 (segment (start 246.25 85.77) (end 246.22 85.74) (width 0.25) (layer "F.Cu") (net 17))
 (segment (start 263.5886 102.29481) (end 266.98019 102.29481) (width 0.25) (layer "F.Cu") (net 19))
 (segment (start 266.98019 102.29481) (end 267.2875 101.9875) (width 0.25) (layer "F.Cu") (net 19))
 (segment (start 263.1314 104.83481) (end 266.98019 104.83481) (width 0.25) (layer "F.Cu") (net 20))
 (segment (start 263.1314 104.83481) (end 263.46621 104.5) (width 0.25) (layer "F.Cu") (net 20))
 (segment (start 266.98019 104.83481) (end 267.2875 104.5275) (width 0.25) (layer "F.Cu") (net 20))
 (segment (start 266.98019 107.37481) (end 267.2875 107.0675) (width 0.25) (layer "F.Cu") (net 21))
 (segment (start 263.5886 107.37481) (end 266.98019 107.37481) (width 0.25) (layer "F.Cu") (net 21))
 (segment (start 263.5886 107.37481) (end 263.5886 107.069936) (width 0.25) (layer "B.Cu") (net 21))
 (segment (start 266.98019 109.91481) (end 267.2875 109.6075) (width 0.25) (layer "F.Cu") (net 22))
 (segment (start 263.1314 109.91481) (end 266.98019 109.91481) (width 0.25) (layer "F.Cu") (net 22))
 (segment (start 263.168794 109.91481) (end 263.168794 109.740545) (width 0.25) (layer "B.Cu") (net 22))
 (segment (start 263.1314 109.91481) (end 263.168794 109.91481) (width 0.25) (layer "B.Cu") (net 22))
 (segment (start 263.5886 112.45481) (end 266.98019 112.45481) (width 0.25) (layer "F.Cu") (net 23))
 (segment (start 266.98019 112.45481) (end 267.2875 112.1475) (width 0.25) (layer "F.Cu") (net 23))
 (segment (start 258.71 100.14) (end 256.34 102.51) (width 0.25) (layer "F.Cu") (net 18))
 (segment (start 256.34 102.51) (end 256.34 103.07481) (width 0.25) (layer "F.Cu") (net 18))
 (segment (start 258.71 94.23981) (end 258.71 100.14) (width 0.25) (layer "F.Cu") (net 18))
 (via (at 258.71 94.23981) (size 0.4) (drill 0.3) (layers "F.Cu" "B.Cu") (free) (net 18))
 (segment (start 262.29621 90.43) (end 263.1314 89.59481) (width 0.25) (layer "B.Cu") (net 18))
 (segment (start 258.71 90.43) (end 262.29621 90.43) (width 0.25) (layer "B.Cu") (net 18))
 (segment (start 258.71 94.23981) (end 258.71 90.43) (width 0.25) (layer "B.Cu") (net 18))
 (segment (start 251.84 112.83) (end 252.35 112.32) (width 0.25) (layer "F.Cu") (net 3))
 (segment (start 253.54 102.64) (end 253.54 97.72481) (width 0.25) (layer "F.Cu") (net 3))
 (segment (start 252.34 112.31) (end 252.35 112.32) (width 0.25) (layer "F.Cu") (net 3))
 (segment (start 251.84 113.51443) (end 251.84 112.83) (width 0.25) (layer "F.Cu") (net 3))
 (segment (start 252.34 104.33) (end 252.34 103.84) (width 0.25) (layer "F.Cu") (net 3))
 (segment (start 252.34 104.33) (end 252.34 112.31) (width 0.25) (layer "F.Cu") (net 3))
 (segment (start 252.34 103.84) (end 253.54 102.64) (width 0.25) (layer "F.Cu") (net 3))
 (via (at 252.35 112.32) (size 0.4) (drill 0.3) (layers "F.Cu" "B.Cu") (free) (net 3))
 (via (at 252.34 104.33) (size 0.4) (drill 0.3) (layers "F.Cu" "B.Cu") (free) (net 3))
 (segment (start 252.76 111.91) (end 259.44 111.91) (width 0.25) (layer "B.Cu") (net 3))
 (segment (start 263.02379 96.65) (end 254.61481 96.65) (width 0.25) (layer "B.Cu") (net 3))
 (segment (start 263.5886 97.21481) (end 263.02379 96.65) (width 0.25) (layer "B.Cu") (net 3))
 (segment (start 252.35 112.32) (end 252.76 111.91) (width 0.25) (layer "B.Cu") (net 3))
 (segment (start 254.34 104.42481) (end 252.43481 104.42481) (width 0.25) (layer "B.Cu") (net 3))
 (segment (start 259.44 113.51443) (end 259.186 113.51443) (width 0.25) (layer "B.Cu") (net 3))
 (segment (start 259.44 111.91) (end 259.44 113.51443) (width 0.25) (layer "B.Cu") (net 3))
 (segment (start 254.61481 96.65) (end 253.54 97.72481) (width 0.25) (layer "B.Cu") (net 3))
 (segment (start 252.43481 104.42481) (end 252.34 104.33) (width 0.25) (layer "B.Cu") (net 3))
 (segment (start 252.34 112.31) (end 252.35 112.32) (width 0.25) (layer "B.Cu") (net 3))
 (segment (start 253.11 113.48481) (end 253.14 113.51481) (width 0.25) (layer "F.Cu") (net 5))
 (segment (start 254.34 101.2) (end 255.89 99.65) (width 0.25) (layer "F.Cu") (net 5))
 (segment (start 254.34 105.82481) (end 253.11519 105.82481) (width 0.25) (layer "F.Cu") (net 5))
 (segment (start 254.34 105.82481) (end 254.34 101.2) (width 0.25) (layer "F.Cu") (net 5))
 (segment (start 255.89 99.65) (end 255.89 98.57481) (width 0.25) (layer "F.Cu") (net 5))
 (segment (start 254.315 105.84981) (end 254.34 105.82481) (width 0.25) (layer "F.Cu") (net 5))
 (segment (start 253.11519 105.82481) (end 253.11 105.83) (width 0.25) (layer "F.Cu") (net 5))
 (segment (start 255.89 98.57481) (end 256.74 97.72481) (width 0.25) (layer "F.Cu") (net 5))
 (segment (start 253.14038 113.51443) (end 253.14 113.51481) (width 0.25) (layer "F.Cu") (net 5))
 (segment (start 254.44 113.51443) (end 253.14038 113.51443) (width 0.25) (layer "F.Cu") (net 5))
 (segment (start 253.11 105.83) (end 253.11 113.48481) (width 0.25) (layer "F.Cu") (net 5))
 (via (at 254.34 105.82481) (size 0.4) (drill 0.3) (layers "F.Cu" "B.Cu") (free) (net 5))
 (via (at 253.14 113.51481) (size 0.4) (drill 0.3) (layers "F.Cu" "B.Cu") (free) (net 5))
 (segment (start 256.74 97.72481) (end 258.14519 99.13) (width 0.25) (layer "B.Cu") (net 5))
 (segment (start 253.14 113.33) (end 253.69 112.78) (width 0.25) (layer "B.Cu") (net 5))
 (segment (start 253.69 112.78) (end 256.20557 112.78) (width 0.25) (layer "B.Cu") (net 5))
 (segment (start 262.50659 99.13) (end 263.1314 99.75481) (width 0.25) (layer "B.Cu") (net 5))
 (segment (start 254.315 105.84981) (end 254.34 105.82481) (width 0.25) (layer "B.Cu") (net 5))
 (segment (start 253.14 113.51481) (end 253.14 113.33) (width 0.25) (layer "B.Cu") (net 5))
 (segment (start 254.315 107.12481) (end 254.315 105.84981) (width 0.25) (layer "B.Cu") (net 5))
 (segment (start 258.14519 99.13) (end 262.50659 99.13) (width 0.25) (layer "B.Cu") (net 5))
 (segment (start 256.20557 112.78) (end 256.94 113.51443) (width 0.25) (layer "B.Cu") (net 5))
 (segment (start 247.8914 92.13481) (end 261.085 92.13481) (width 0.25) (layer "F.Cu") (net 25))
 (segment (start 261.085 119.492) (end 263.625 122.032) (width 0.25) (layer "F.Cu") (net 25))
 (segment (start 261.085 92.13481) (end 261.085 119.492) (width 0.25) (layer "F.Cu") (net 25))
 (segment (start 259.44 118.72481) (end 259.44 114.51519) (width 0.25) (layer "F.Cu") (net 16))
 (segment (start 259.44 118.72481) (end 259.44 114.51519) (width 0.25) (layer "B.Cu") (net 16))
 (segment (start 256.9 114.55519) (end 256.94 114.51519) (width 0.25) (layer "F.Cu") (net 1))
 (segment (start 256.9 118.72481) (end 256.9 114.55519) (width 0.25) (layer "F.Cu") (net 1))
 (segment (start 256.9 118.72481) (end 256.9 114.55519) (width 0.25) (layer "B.Cu") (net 1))
 (segment (start 256.9 114.55519) (end 256.94 114.51519) (width 0.25) (layer "B.Cu") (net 1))
 (segment (start 254.44 114.51519) (end 254.44 118.64481) (width 0.25) (layer "F.Cu") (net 15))
 (segment (start 254.44 118.64481) (end 254.36 118.72481) (width 0.25) (layer "F.Cu") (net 15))
 (segment (start 254.36 118.72481) (end 254.36 114.59519) (width 0.25) (layer "B.Cu") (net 15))
 (segment (start 254.36 114.59519) (end 254.44 114.51519) (width 0.25) (layer "B.Cu") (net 15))
 (segment (start 251.84 118.70481) (end 251.82 118.72481) (width 0.25) (layer "F.Cu") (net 4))
 (segment (start 251.84 114.51519) (end 251.84 118.70481) (width 0.25) (layer "F.Cu") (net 4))
 (segment (start 251.82 114.53519) (end 251.84 114.51519) (width 0.25) (layer "B.Cu") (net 4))
 (segment (start 251.82 118.72481) (end 251.82 114.53519) (width 0.25) (layer "B.Cu") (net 4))
 (segment (start 257.95 108.00962) (end 257.95 118.274362) (width 0.25) (layer "F.Cu") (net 7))
 (segment (start 257.92 119.152258) (end 257.92 122.99019) (width 0.25) (layer "F.Cu") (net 7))
 (segment (start 257.95 118.274362) (end 257.9235 118.300862) (width 0.25) (layer "F.Cu") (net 7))
 (segment (start 258.04181 123.11519) (end 258.04181 125.459039) (width 0.25) (layer "F.Cu") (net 7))
 (segment (start 257.92 122.99019) (end 258.045 123.11519) (width 0.25) (layer "F.Cu") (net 7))
 (segment (start 257.9235 119.148758) (end 257.92 119.152258) (width 0.25) (layer "F.Cu") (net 7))
 (segment (start 257.9235 118.300862) (end 257.9235 119.148758) (width 0.25) (layer "F.Cu") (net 7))
 (segment (start 258.04181 125.459039) (end 255.9 127.600849) (width 0.25) (layer "F.Cu") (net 7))
 (segment (start 255.9 127.600849) (end 255.9 130.83) (width 0.25) (layer "F.Cu") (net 7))
 (segment (start 257.06519 107.12481) (end 257.95 108.00962) (width 0.25) (layer "F.Cu") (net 7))
 (via (at 257.06519 107.12481) (size 0.4) (drill 0.3) (layers "F.Cu" "B.Cu") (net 7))
 (segment (start 257.06519 107.12481) (end 255.765 107.12481) (width 0.25) (layer "B.Cu") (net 7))
 (segment (start 258.4 104.56) (end 258.4 122.199782) (width 0.25) (layer "F.Cu") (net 8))
 (segment (start 260.415208 128.854792) (end 258.44 130.83) (width 0.25) (layer "F.Cu") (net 8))
 (segment (start 258.44 104.52) (end 258.4 104.56) (width 0.25) (layer "F.Cu") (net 8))
 (segment (start 258.29481 104.37481) (end 258.44 104.52) (width 0.25) (layer "F.Cu") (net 8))
 (segment (start 260.415208 124.21499) (end 260.415208 128.854792) (width 0.25) (layer "F.Cu") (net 8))
 (segment (start 258.4 122.199782) (end 260.415208 124.21499) (width 0.25) (layer "F.Cu") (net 8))
 (segment (start 256.34 104.37481) (end 258.29481 104.37481) (width 0.25) (layer "F.Cu") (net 8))
 (via (at 258.44 104.52) (size 0.4) (drill 0.3) (layers "F.Cu" "B.Cu") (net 8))
 (segment (start 258.34481 104.42481) (end 258.44 104.52) (width 0.25) (layer "B.Cu") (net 8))
 (segment (start 255.79 104.42481) (end 258.34481 104.42481) (width 0.25) (layer "B.Cu") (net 8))
 (segment (start 263.1314 114.99481) (end 266.98019 114.99481) (width 0.25) (layer "F.Cu") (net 24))
 (segment (start 266.98019 114.99481) (end 267.2875 114.6875) (width 0.25) (layer "F.Cu") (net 24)))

